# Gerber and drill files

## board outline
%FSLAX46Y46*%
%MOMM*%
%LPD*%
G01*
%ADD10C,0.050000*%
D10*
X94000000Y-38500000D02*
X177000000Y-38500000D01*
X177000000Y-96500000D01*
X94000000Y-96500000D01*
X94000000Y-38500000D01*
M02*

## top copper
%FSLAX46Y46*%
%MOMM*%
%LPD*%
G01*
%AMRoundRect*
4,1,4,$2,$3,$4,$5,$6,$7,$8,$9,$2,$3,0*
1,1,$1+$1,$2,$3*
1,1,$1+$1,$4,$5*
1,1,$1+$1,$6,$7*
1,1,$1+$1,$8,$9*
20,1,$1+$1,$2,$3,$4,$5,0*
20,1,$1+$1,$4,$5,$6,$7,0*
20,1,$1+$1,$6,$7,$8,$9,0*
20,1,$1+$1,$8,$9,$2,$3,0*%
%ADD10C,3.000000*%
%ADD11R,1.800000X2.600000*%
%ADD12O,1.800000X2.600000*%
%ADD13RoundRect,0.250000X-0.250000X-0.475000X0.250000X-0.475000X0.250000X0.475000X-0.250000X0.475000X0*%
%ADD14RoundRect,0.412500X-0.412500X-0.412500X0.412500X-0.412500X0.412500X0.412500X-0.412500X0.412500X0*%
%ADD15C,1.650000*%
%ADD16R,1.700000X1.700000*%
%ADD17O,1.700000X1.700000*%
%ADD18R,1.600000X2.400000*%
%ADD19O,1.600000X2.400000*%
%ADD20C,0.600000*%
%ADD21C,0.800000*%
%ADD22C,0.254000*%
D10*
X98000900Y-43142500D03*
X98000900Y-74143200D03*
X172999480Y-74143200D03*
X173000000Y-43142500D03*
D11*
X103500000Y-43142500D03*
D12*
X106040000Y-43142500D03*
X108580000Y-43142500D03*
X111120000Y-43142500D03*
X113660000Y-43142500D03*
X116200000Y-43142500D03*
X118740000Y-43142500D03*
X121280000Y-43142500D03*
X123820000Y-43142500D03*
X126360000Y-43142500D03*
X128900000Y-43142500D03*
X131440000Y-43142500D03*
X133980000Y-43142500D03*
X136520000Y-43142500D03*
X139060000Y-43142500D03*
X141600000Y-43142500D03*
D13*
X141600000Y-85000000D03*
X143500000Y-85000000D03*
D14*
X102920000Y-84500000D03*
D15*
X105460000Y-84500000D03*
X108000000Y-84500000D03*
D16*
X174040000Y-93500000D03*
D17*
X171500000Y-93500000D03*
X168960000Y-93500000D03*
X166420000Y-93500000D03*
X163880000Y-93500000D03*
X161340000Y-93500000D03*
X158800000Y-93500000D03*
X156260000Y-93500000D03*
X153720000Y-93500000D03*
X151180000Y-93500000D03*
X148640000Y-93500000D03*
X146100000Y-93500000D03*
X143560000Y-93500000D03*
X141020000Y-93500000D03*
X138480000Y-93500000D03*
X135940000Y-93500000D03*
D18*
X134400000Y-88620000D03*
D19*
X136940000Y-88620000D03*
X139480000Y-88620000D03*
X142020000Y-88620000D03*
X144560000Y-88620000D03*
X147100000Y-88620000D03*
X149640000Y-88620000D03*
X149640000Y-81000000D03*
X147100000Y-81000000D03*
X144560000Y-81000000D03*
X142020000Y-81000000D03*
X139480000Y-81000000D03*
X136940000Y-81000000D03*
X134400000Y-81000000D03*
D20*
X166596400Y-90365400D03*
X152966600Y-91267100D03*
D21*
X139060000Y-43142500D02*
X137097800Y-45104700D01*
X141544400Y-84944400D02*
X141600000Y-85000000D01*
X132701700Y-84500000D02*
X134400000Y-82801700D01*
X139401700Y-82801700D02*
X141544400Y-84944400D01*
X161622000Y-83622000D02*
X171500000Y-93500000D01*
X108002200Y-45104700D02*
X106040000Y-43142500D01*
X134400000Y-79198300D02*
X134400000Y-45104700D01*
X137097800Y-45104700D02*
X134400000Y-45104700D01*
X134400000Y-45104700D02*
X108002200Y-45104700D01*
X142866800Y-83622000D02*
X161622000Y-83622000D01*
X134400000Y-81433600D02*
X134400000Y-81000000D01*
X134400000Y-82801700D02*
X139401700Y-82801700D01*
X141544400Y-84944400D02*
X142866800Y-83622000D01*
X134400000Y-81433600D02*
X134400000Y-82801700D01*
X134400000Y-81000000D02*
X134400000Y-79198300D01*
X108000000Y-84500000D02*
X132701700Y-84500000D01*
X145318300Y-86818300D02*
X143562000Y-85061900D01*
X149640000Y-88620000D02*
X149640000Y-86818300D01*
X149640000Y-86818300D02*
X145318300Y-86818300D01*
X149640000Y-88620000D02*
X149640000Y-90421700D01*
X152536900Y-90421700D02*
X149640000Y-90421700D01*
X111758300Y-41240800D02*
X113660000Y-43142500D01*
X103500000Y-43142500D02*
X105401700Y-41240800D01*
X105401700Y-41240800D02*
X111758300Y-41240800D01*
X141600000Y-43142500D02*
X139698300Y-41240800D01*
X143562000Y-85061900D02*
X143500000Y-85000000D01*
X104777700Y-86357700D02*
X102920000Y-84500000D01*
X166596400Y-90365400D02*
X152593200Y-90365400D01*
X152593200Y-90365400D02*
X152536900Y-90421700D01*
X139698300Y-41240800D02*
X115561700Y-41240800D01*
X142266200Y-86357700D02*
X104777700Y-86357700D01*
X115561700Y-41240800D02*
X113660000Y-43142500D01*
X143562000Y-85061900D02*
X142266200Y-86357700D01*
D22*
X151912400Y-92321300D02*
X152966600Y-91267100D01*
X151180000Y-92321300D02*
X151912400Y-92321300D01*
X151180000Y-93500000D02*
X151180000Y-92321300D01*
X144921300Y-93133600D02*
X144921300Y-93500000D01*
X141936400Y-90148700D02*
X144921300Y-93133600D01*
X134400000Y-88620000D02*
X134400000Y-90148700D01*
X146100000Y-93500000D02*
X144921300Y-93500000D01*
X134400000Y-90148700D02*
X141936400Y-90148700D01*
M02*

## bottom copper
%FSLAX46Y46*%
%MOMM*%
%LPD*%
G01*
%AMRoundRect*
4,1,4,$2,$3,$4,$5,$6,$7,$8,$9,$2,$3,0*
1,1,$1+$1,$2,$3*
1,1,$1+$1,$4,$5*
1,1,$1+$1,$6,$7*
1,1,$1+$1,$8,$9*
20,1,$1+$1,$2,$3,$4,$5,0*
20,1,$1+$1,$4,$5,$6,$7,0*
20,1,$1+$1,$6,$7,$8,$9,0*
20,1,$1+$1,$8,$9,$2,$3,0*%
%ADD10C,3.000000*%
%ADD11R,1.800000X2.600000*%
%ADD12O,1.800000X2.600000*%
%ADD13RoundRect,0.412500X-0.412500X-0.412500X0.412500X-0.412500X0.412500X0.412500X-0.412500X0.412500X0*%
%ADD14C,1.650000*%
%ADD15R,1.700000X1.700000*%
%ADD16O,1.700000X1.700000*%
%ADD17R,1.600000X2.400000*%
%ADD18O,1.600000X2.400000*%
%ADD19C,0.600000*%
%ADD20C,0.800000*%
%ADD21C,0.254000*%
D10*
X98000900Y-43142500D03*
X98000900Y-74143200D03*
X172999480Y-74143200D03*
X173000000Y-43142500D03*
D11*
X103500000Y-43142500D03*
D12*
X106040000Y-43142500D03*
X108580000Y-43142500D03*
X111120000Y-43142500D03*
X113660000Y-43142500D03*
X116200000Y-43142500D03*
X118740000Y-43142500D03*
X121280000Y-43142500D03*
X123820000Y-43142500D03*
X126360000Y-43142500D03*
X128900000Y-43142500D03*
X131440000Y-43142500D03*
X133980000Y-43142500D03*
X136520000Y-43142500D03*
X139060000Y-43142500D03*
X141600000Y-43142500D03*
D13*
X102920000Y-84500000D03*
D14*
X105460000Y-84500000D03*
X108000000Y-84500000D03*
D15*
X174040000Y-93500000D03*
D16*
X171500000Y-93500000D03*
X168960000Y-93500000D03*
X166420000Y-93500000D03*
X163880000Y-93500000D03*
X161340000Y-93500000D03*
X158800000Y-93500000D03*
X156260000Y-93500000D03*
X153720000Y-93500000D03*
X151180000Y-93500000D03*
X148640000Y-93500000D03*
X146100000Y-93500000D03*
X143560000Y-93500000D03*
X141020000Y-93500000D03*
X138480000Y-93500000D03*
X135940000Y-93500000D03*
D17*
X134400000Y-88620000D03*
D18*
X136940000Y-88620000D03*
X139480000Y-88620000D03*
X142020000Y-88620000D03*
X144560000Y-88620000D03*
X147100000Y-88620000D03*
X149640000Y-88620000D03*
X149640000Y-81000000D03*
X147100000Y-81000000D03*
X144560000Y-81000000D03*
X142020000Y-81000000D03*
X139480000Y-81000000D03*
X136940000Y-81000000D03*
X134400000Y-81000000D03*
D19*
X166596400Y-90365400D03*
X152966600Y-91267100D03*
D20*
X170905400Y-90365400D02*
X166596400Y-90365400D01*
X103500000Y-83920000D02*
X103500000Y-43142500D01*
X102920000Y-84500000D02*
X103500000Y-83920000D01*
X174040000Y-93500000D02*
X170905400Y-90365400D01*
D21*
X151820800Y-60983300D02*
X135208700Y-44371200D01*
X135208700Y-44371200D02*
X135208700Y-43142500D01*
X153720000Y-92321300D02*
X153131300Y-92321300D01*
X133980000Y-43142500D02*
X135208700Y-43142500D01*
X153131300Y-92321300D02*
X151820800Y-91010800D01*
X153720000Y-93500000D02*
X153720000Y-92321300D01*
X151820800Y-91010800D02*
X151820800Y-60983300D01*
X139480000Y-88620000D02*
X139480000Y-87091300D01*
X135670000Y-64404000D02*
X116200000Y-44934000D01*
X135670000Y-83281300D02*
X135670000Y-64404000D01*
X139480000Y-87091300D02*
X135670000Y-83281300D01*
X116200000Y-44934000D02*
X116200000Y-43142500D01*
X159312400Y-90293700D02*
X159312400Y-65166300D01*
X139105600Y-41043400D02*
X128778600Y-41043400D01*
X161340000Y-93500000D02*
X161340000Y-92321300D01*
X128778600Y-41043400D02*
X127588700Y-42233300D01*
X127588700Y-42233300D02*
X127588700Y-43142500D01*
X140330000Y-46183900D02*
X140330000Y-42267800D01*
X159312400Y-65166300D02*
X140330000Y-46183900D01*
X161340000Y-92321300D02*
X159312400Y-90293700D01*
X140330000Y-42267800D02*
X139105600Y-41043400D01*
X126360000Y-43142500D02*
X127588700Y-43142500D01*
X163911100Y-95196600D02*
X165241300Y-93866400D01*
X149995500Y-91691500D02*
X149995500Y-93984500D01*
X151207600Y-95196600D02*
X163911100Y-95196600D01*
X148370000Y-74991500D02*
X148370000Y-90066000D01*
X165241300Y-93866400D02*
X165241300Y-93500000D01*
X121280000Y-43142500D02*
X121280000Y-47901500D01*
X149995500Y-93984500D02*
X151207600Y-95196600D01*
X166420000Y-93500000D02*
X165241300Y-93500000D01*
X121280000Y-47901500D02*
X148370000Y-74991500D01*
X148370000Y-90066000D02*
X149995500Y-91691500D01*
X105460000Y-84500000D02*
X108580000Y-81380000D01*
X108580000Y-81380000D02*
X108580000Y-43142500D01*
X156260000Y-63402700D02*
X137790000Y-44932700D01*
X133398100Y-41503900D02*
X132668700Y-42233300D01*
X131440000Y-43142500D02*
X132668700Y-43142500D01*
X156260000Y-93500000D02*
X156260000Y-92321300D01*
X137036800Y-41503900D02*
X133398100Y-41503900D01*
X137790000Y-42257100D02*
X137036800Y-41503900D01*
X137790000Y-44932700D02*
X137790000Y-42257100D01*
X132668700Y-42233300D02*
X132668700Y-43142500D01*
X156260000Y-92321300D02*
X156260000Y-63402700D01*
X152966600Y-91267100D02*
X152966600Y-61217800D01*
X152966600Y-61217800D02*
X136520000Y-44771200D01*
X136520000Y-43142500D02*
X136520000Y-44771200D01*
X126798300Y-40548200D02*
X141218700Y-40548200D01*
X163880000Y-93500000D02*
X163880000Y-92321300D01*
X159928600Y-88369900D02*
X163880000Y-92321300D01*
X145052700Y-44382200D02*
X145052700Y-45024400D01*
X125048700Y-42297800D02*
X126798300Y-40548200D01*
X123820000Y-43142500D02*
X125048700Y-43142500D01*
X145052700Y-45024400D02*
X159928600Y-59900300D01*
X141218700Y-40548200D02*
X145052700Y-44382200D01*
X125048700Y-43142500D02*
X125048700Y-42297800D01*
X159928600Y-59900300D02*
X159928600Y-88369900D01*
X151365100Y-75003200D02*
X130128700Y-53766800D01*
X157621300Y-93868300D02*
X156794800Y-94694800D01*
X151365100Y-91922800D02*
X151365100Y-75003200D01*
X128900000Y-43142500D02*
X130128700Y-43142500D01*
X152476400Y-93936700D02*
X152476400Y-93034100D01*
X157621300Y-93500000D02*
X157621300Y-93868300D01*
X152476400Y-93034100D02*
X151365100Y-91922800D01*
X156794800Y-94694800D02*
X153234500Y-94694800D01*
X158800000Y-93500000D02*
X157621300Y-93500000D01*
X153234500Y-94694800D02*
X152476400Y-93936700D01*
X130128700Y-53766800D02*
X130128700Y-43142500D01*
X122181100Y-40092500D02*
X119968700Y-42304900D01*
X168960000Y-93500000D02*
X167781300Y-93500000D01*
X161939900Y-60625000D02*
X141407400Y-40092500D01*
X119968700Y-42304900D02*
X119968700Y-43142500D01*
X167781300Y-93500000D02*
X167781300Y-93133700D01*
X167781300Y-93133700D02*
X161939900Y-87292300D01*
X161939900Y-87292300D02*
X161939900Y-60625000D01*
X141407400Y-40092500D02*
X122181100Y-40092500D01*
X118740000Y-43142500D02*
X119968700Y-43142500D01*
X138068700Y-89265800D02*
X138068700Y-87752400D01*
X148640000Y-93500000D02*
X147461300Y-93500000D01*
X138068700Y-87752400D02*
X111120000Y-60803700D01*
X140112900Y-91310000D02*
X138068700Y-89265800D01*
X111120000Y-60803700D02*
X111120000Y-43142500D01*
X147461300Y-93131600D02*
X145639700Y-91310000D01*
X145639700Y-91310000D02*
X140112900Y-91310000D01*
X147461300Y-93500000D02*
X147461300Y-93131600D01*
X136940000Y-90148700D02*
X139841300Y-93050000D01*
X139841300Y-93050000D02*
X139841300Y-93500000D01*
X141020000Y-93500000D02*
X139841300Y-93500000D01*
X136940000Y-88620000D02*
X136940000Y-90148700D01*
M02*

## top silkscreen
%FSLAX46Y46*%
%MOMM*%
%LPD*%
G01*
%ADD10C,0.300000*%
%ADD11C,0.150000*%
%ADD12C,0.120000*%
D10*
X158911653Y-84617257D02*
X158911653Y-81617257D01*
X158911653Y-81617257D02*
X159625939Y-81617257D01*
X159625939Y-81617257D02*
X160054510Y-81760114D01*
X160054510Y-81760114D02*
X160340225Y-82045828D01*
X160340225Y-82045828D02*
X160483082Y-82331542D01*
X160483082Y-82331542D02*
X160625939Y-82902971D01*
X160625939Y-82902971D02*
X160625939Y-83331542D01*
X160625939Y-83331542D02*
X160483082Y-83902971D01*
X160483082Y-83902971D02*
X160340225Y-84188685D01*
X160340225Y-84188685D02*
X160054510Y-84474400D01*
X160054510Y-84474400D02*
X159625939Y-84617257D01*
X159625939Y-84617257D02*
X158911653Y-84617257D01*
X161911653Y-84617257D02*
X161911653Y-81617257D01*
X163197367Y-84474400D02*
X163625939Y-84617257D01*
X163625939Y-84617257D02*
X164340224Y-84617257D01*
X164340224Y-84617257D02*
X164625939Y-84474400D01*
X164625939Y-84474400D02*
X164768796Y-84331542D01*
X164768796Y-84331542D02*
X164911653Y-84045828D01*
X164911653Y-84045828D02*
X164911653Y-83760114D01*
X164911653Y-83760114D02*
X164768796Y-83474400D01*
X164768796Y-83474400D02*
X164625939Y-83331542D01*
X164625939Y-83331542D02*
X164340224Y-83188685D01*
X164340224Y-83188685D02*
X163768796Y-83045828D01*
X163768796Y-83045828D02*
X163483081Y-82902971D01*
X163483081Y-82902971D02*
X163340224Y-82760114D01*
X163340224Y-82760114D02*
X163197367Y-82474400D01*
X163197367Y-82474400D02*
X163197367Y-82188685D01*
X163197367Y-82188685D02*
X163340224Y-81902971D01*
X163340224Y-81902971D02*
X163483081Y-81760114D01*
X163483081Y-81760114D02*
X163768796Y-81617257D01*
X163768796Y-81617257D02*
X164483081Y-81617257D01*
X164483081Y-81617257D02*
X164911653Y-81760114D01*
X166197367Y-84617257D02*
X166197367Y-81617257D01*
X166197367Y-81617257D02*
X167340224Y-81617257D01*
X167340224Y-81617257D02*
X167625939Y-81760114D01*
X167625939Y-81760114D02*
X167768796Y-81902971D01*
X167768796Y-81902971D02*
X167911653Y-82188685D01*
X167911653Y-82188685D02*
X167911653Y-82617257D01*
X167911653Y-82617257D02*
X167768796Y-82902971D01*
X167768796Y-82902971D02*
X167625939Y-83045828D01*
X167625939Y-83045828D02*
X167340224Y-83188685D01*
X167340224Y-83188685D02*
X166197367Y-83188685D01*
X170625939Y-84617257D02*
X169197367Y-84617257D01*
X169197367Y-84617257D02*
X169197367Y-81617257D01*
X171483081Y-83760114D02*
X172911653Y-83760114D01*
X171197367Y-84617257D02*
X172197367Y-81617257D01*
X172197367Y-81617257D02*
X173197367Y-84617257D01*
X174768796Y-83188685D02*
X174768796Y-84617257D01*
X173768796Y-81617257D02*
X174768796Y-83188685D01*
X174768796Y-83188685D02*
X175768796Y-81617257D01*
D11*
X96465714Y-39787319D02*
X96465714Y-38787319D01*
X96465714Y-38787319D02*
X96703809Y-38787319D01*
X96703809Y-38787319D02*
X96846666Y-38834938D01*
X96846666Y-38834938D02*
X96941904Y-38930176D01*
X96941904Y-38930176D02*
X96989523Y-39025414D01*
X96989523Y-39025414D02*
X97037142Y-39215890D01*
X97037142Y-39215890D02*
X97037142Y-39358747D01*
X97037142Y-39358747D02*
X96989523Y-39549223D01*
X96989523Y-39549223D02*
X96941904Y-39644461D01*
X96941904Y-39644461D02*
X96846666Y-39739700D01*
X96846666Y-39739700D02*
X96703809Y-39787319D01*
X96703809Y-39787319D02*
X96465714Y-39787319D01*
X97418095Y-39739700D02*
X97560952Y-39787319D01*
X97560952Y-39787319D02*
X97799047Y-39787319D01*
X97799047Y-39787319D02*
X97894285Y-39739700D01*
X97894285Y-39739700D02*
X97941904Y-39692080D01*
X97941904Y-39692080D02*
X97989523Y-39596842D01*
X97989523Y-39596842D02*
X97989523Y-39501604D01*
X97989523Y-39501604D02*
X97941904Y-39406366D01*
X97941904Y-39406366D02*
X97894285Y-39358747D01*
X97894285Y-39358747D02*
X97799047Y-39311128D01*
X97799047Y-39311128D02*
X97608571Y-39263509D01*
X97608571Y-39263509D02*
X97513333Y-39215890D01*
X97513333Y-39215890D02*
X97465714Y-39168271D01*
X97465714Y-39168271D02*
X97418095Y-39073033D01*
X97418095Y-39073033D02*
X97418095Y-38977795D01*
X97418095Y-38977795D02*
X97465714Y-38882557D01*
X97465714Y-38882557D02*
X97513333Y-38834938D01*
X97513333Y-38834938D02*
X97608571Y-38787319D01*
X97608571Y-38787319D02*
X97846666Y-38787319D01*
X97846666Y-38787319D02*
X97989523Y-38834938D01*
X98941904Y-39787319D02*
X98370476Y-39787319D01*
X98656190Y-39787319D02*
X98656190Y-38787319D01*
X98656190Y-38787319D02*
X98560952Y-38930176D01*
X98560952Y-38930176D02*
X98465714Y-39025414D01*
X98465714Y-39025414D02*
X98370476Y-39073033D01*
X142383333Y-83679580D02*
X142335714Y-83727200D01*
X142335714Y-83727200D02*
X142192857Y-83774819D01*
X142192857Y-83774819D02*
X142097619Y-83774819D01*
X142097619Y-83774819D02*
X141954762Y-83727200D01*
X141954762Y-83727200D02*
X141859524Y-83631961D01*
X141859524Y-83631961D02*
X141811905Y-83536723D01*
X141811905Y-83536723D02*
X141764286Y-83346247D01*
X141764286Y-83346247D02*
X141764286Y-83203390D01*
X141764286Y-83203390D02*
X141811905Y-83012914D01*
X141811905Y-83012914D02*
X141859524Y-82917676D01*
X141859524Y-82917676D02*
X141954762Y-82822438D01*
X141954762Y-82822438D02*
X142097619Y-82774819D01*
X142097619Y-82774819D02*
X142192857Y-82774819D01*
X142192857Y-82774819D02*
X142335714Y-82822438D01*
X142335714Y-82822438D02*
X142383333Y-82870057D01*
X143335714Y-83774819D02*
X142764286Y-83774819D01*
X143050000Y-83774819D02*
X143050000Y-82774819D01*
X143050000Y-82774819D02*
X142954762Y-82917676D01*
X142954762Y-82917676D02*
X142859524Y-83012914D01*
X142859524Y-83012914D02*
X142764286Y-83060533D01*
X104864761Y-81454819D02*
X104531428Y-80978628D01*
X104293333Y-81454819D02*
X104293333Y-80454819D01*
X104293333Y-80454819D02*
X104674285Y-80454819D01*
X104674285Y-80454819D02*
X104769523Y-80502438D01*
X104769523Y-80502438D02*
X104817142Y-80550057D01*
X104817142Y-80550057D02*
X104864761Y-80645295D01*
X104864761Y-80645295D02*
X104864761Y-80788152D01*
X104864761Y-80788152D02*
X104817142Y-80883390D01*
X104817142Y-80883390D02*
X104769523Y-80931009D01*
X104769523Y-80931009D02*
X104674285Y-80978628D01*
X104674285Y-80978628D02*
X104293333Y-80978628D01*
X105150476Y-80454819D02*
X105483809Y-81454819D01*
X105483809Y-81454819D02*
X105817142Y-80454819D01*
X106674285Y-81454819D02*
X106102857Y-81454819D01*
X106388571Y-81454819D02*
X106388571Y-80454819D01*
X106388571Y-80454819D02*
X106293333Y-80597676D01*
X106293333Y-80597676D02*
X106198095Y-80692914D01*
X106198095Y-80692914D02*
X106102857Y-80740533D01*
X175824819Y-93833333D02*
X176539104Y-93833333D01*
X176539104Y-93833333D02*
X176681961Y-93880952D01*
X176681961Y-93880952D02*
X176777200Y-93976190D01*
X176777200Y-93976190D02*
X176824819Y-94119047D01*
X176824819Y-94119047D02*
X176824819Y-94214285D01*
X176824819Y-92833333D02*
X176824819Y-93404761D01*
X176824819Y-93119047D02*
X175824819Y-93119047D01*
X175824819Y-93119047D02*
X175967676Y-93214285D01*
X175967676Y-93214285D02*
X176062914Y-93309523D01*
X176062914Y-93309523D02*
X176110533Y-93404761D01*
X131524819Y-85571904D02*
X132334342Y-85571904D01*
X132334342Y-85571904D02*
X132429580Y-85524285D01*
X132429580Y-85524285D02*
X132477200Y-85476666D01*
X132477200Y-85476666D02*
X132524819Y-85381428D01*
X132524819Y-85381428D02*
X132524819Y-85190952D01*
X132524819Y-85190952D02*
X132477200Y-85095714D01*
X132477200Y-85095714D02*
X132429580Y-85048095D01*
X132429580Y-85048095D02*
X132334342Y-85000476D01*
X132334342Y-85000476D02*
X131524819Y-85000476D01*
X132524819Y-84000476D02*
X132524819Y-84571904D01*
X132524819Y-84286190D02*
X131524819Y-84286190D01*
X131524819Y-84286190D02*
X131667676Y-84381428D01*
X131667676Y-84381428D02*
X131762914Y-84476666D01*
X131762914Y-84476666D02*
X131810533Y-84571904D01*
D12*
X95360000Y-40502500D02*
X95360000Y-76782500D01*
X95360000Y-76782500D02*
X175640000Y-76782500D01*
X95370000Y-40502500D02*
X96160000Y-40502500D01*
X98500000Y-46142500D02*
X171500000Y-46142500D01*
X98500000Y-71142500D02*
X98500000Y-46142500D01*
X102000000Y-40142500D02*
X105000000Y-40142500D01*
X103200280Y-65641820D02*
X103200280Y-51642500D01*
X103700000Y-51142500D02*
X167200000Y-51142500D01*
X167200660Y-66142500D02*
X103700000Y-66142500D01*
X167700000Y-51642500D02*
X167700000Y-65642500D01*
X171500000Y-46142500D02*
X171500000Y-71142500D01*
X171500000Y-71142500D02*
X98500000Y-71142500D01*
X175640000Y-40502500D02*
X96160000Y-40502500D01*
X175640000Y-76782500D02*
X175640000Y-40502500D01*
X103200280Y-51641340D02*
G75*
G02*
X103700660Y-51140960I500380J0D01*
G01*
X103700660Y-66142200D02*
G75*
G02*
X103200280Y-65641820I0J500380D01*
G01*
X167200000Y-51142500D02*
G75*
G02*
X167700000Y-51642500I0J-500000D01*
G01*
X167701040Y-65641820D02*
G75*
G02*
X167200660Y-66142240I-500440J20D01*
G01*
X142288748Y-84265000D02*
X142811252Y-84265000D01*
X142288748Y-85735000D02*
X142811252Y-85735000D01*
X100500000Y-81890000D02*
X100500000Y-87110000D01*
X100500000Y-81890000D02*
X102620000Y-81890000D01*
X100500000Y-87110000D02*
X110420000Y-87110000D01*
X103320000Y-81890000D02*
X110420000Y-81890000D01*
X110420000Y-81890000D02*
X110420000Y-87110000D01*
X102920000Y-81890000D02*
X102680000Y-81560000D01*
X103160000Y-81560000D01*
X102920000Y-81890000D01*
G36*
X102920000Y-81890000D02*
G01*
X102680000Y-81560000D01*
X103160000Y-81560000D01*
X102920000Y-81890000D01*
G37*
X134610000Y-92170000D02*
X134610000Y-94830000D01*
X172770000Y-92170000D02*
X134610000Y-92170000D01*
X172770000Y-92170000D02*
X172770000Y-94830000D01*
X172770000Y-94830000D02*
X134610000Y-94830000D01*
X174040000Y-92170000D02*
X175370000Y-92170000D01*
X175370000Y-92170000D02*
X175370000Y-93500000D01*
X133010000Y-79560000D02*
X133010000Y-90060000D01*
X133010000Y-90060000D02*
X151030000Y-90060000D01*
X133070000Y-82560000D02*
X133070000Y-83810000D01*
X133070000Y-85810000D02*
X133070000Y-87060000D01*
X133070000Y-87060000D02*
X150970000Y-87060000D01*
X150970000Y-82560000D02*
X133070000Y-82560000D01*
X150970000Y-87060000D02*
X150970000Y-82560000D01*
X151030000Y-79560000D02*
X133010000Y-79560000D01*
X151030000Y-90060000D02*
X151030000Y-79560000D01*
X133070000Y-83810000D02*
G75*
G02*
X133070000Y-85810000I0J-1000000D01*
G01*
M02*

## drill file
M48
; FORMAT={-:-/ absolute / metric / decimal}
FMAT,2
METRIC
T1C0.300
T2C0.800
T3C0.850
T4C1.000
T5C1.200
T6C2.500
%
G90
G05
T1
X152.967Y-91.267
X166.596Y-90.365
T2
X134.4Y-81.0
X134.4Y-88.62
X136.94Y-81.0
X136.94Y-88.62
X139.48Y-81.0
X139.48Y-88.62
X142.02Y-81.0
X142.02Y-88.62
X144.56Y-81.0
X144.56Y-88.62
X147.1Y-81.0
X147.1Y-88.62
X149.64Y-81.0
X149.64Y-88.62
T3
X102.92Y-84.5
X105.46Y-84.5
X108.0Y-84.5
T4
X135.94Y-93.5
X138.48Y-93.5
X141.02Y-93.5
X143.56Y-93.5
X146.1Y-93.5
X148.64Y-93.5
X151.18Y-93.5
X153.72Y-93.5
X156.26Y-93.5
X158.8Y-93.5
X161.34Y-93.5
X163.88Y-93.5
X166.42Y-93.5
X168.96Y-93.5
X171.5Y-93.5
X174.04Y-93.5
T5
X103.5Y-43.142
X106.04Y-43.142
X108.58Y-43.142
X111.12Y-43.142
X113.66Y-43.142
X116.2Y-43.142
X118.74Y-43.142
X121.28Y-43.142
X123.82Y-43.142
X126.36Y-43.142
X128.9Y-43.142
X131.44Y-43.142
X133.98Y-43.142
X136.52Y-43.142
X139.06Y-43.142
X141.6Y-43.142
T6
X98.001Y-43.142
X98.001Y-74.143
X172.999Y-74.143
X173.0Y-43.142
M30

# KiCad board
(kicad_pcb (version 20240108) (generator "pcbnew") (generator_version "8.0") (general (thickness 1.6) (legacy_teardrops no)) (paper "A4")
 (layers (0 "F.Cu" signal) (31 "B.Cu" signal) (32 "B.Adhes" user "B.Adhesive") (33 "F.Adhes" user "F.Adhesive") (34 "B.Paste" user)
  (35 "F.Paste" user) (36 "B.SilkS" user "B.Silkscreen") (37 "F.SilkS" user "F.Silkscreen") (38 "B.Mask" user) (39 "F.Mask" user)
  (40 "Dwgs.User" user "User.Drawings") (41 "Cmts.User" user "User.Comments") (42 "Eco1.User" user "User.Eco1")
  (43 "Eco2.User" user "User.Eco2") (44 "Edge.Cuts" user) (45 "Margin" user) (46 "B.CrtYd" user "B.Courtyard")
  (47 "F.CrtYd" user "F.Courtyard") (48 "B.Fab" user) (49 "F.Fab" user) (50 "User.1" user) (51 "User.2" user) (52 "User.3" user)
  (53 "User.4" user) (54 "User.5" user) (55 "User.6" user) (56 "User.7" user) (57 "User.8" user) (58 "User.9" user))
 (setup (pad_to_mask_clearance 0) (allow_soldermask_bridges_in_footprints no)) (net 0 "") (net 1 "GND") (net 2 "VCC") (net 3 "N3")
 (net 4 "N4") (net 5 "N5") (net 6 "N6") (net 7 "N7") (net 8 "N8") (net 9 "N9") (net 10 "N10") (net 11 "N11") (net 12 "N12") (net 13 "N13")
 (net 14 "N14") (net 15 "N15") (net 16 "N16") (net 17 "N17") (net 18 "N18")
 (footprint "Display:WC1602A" (layer "F.Cu") (at 103.5 43.1425)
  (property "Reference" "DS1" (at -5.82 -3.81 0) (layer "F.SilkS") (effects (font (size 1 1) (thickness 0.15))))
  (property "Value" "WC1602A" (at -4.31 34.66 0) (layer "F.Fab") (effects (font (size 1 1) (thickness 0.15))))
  (fp_line (start -8.14 -2.64) (end -8.14 33.64) (stroke (width 0.12) (type solid)) (layer "F.SilkS"))
  (fp_line (start -8.14 33.64) (end 72.14 33.64) (stroke (width 0.12) (type solid)) (layer "F.SilkS"))
  (fp_line (start -8.13 -2.64) (end -7.34 -2.64) (stroke (width 0.12) (type solid)) (layer "F.SilkS"))
  (fp_line (start -5 3) (end 68 3) (stroke (width 0.12) (type solid)) (layer "F.SilkS"))
  (fp_line (start -5 28) (end -5 3) (stroke (width 0.12) (type solid)) (layer "F.SilkS"))
  (fp_line (start -1.5 -3) (end 1.5 -3) (stroke (width 0.12) (type solid)) (layer "F.SilkS"))
  (fp_line (start -0.29972 22.49932) (end -0.29972 8.5) (stroke (width 0.12) (type solid)) (layer "F.SilkS"))
  (fp_line (start 0.2 8) (end 63.7 8) (stroke (width 0.12) (type solid)) (layer "F.SilkS"))
  (fp_line (start 63.70066 23) (end 0.2 23) (stroke (width 0.12) (type solid)) (layer "F.SilkS"))
  (fp_line (start 64.2 8.5) (end 64.2 22.5) (stroke (width 0.12) (type solid)) (layer "F.SilkS"))
  (fp_line (start 68 3) (end 68 28) (stroke (width 0.12) (type solid)) (layer "F.SilkS"))
  (fp_line (start 68 28) (end -5 28) (stroke (width 0.12) (type solid)) (layer "F.SilkS"))
  (fp_line (start 72.14 -2.64) (end -7.34 -2.64) (stroke (width 0.12) (type solid)) (layer "F.SilkS"))
  (fp_line (start 72.14 33.64) (end 72.14 -2.64) (stroke (width 0.12) (type solid)) (layer "F.SilkS"))
  (fp_arc (start -0.29972 8.49884) (mid -0.153162 8.145018) (end 0.20066 7.99846) (stroke (width 0.12) (type solid)) (layer "F.SilkS"))
  (fp_arc (start 0.20066 22.9997) (mid -0.153162 22.853142) (end -0.29972 22.49932) (stroke (width 0.12) (type solid)) (layer "F.SilkS"))
  (fp_arc (start 63.7 8) (mid 64.053553 8.146447) (end 64.2 8.5) (stroke (width 0.12) (type solid)) (layer "F.SilkS"))
  (fp_arc (start 64.20104 22.49932) (mid 64.054473 22.853115) (end 63.70066 22.9997) (stroke (width 0.12) (type solid)) (layer "F.SilkS"))
  (pad "" thru_hole circle (at -5.4991 0) (size 3 3) (drill 2.5) (layers "*.Cu" "*.Mask") (remove_unused_layers no))
  (pad "" thru_hole circle (at -5.4991 31.0007) (size 3 3) (drill 2.5) (layers "*.Cu" "*.Mask") (remove_unused_layers no))
  (pad "" thru_hole circle (at 69.49948 31.0007) (size 3 3) (drill 2.5) (layers "*.Cu" "*.Mask") (remove_unused_layers no))
  (pad "" thru_hole circle (at 69.5 0) (size 3 3) (drill 2.5) (layers "*.Cu" "*.Mask") (remove_unused_layers no))
  (pad "1" thru_hole rect (at 0 0) (size 1.8 2.6) (drill 1.2) (layers "*.Cu" "*.Mask") (remove_unused_layers no) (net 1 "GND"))
  (pad "2" thru_hole oval (at 2.54 0) (size 1.8 2.6) (drill 1.2) (layers "*.Cu" "*.Mask") (remove_unused_layers no) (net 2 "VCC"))
  (pad "3" thru_hole oval (at 5.08 0) (size 1.8 2.6) (drill 1.2) (layers "*.Cu" "*.Mask") (remove_unused_layers no) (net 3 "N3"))
  (pad "4" thru_hole oval (at 7.62 0) (size 1.8 2.6) (drill 1.2) (layers "*.Cu" "*.Mask") (remove_unused_layers no) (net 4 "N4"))
  (pad "5" thru_hole oval (at 10.16 0) (size 1.8 2.6) (drill 1.2) (layers "*.Cu" "*.Mask") (remove_unused_layers no) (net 1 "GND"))
  (pad "6" thru_hole oval (at 12.7 0) (size 1.8 2.6) (drill 1.2) (layers "*.Cu" "*.Mask") (remove_unused_layers no) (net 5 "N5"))
  (pad "7" thru_hole oval (at 15.24 0) (size 1.8 2.6) (drill 1.2) (layers "*.Cu" "*.Mask") (remove_unused_layers no) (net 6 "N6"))
  (pad "8" thru_hole oval (at 17.78 0) (size 1.8 2.6) (drill 1.2) (layers "*.Cu" "*.Mask") (remove_unused_layers no) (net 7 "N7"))
  (pad "9" thru_hole oval (at 20.32 0) (size 1.8 2.6) (drill 1.2) (layers "*.Cu" "*.Mask") (remove_unused_layers no) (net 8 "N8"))
  (pad "10" thru_hole oval (at 22.86 0) (size 1.8 2.6) (drill 1.2) (layers "*.Cu" "*.Mask") (remove_unused_layers no) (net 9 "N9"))
  (pad "11" thru_hole oval (at 25.4 0) (size 1.8 2.6) (drill 1.2) (layers "*.Cu" "*.Mask") (remove_unused_layers no) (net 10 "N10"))
  (pad "12" thru_hole oval (at 27.94 0) (size 1.8 2.6) (drill 1.2) (layers "*.Cu" "*.Mask") (remove_unused_layers no) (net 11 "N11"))
  (pad "13" thru_hole oval (at 30.48 0) (size 1.8 2.6) (drill 1.2) (layers "*.Cu" "*.Mask") (remove_unused_layers no) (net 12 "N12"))
  (pad "14" thru_hole oval (at 33.02 0) (size 1.8 2.6) (drill 1.2) (layers "*.Cu" "*.Mask") (remove_unused_layers no) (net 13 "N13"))
  (pad "15" thru_hole oval (at 35.56 0) (size 1.8 2.6) (drill 1.2) (layers "*.Cu" "*.Mask") (remove_unused_layers no) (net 2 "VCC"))
  (pad "16" thru_hole oval (at 38.1 0) (size 1.8 2.6) (drill 1.2) (layers "*.Cu" "*.Mask") (remove_unused_layers no) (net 1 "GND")))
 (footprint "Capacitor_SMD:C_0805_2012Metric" (layer "F.Cu") (at 142.55 85)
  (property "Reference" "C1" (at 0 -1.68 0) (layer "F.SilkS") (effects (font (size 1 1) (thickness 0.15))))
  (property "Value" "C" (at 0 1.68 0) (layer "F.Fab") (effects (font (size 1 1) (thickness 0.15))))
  (fp_line (start -0.261252 -0.735) (end 0.261252 -0.735) (stroke (width 0.12) (type solid)) (layer "F.SilkS"))
  (fp_line (start -0.261252 0.735) (end 0.261252 0.735) (stroke (width 0.12) (type solid)) (layer "F.SilkS"))
  (pad "1" smd roundrect (at -0.95 0) (size 1 1.45) (layers "F.Cu" "F.Paste" "F.Mask") (roundrect_rratio 0.25) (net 2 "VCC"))
  (pad "2" smd roundrect (at 0.95 0) (size 1 1.45) (layers "F.Cu" "F.Paste" "F.Mask") (roundrect_rratio 0.25) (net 1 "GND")))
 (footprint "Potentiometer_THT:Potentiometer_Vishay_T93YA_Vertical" (layer "F.Cu") (at 102.92 84.5)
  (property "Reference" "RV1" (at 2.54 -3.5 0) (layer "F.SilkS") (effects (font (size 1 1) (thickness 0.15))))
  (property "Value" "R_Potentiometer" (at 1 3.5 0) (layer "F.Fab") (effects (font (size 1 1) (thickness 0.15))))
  (fp_line (start -2.42 -2.61) (end -2.42 2.61) (stroke (width 0.12) (type default)) (layer "F.SilkS"))
  (fp_line (start -2.42 -2.61) (end -0.3 -2.61) (stroke (width 0.12) (type default)) (layer "F.SilkS"))
  (fp_line (start -2.42 2.61) (end 7.5 2.61) (stroke (width 0.12) (type default)) (layer "F.SilkS"))
  (fp_line (start 0.4 -2.61) (end 7.5 -2.61) (stroke (width 0.12) (type default)) (layer "F.SilkS"))
  (fp_line (start 7.5 -2.61) (end 7.5 2.61) (stroke (width 0.12) (type default)) (layer "F.SilkS"))
  (fp_poly
   (pts (xy 0 -2.61) (xy -0.24 -2.94) (xy 0.24 -2.94) (xy 0 -2.61)) (stroke (width 0.12) (type solid)) (fill solid) (layer "F.SilkS"))
  (pad "1" thru_hole roundrect (at 0 0) (size 1.65 1.65) (drill 0.85) (layers "*.Cu" "*.Mask") (remove_unused_layers no)
   (roundrect_rratio 0.25) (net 1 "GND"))
  (pad "2" thru_hole circle (at 2.54 0) (size 1.65 1.65) (drill 0.85) (layers "*.Cu" "*.Mask") (remove_unused_layers no) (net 3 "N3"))
  (pad "3" thru_hole circle (at 5.08 0) (size 1.65 1.65) (drill 0.85) (layers "*.Cu" "*.Mask") (remove_unused_layers no) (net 2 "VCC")))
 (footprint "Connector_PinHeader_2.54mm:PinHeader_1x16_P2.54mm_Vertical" (layer "F.Cu") (at 174.04 93.5 -90)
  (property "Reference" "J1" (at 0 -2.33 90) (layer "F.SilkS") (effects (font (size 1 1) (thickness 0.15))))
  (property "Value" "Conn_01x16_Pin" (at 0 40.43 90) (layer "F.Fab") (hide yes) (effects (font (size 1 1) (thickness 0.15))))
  (fp_line (start -1.33 39.43) (end 1.33 39.43) (stroke (width 0.12) (type solid)) (layer "F.SilkS"))
  (fp_line (start -1.33 1.27) (end -1.33 39.43) (stroke (width 0.12) (type solid)) (layer "F.SilkS"))
  (fp_line (start -1.33 1.27) (end 1.33 1.27) (stroke (width 0.12) (type solid)) (layer "F.SilkS"))
  (fp_line (start 1.33 1.27) (end 1.33 39.43) (stroke (width 0.12) (type solid)) (layer "F.SilkS"))
  (fp_line (start -1.33 0) (end -1.33 -1.33) (stroke (width 0.12) (type solid)) (layer "F.SilkS"))
  (fp_line (start -1.33 -1.33) (end 0 -1.33) (stroke (width 0.12) (type solid)) (layer "F.SilkS"))
  (pad "1" thru_hole rect (at 0 0 270) (size 1.7 1.7) (drill 1) (layers "*.Cu" "*.Mask") (remove_unused_layers no) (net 1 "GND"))
  (pad "2" thru_hole oval (at 0 2.54 270) (size 1.7 1.7) (drill 1) (layers "*.Cu" "*.Mask") (remove_unused_layers no) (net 2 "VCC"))
  (pad "3" thru_hole oval (at 0 5.08 270) (size 1.7 1.7) (drill 1) (layers "*.Cu" "*.Mask") (remove_unused_layers no) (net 6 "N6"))
  (pad "4" thru_hole oval (at 0 7.62 270) (size 1.7 1.7) (drill 1) (layers "*.Cu" "*.Mask") (remove_unused_layers no) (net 7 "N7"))
  (pad "5" thru_hole oval (at 0 10.16 270) (size 1.7 1.7) (drill 1) (layers "*.Cu" "*.Mask") (remove_unused_layers no) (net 8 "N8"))
  (pad "6" thru_hole oval (at 0 12.7 270) (size 1.7 1.7) (drill 1) (layers "*.Cu" "*.Mask") (remove_unused_layers no) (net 9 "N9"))
  (pad "7" thru_hole oval (at 0 15.24 270) (size 1.7 1.7) (drill 1) (layers "*.Cu" "*.Mask") (remove_unused_layers no) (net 10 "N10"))
  (pad "8" thru_hole oval (at 0 17.78 270) (size 1.7 1.7) (drill 1) (layers "*.Cu" "*.Mask") (remove_unused_layers no) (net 11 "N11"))
  (pad "9" thru_hole oval (at 0 20.32 270) (size 1.7 1.7) (drill 1) (layers "*.Cu" "*.Mask") (remove_unused_layers no) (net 12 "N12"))
  (pad "10" thru_hole oval (at 0 22.86 270) (size 1.7 1.7) (drill 1) (layers "*.Cu" "*.Mask") (remove_unused_layers no) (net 13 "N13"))
  (pad "11" thru_hole oval (at 0 25.4 270) (size 1.7 1.7) (drill 1) (layers "*.Cu" "*.Mask") (remove_unused_layers no) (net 4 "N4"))
  (pad "12" thru_hole oval (at 0 27.94 270) (size 1.7 1.7) (drill 1) (layers "*.Cu" "*.Mask") (remove_unused_layers no) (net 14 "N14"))
  (pad "13" thru_hole oval (at 0 30.48 270) (size 1.7 1.7) (drill 1) (layers "*.Cu" "*.Mask") (remove_unused_layers no) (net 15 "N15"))
  (pad "14" thru_hole oval (at 0 33.02 270) (size 1.7 1.7) (drill 1) (layers "*.Cu" "*.Mask") (remove_unused_layers no) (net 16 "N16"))
  (pad "15" thru_hole oval (at 0 35.56 270) (size 1.7 1.7) (drill 1) (layers "*.Cu" "*.Mask") (remove_unused_layers no) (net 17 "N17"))
  (pad "16" thru_hole oval (at 0 38.1 270) (size 1.7 1.7) (drill 1) (layers "*.Cu" "*.Mask") (remove_unused_layers no) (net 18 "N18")))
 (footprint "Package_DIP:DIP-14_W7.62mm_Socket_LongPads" (layer "F.Cu") (at 134.4 88.62 90)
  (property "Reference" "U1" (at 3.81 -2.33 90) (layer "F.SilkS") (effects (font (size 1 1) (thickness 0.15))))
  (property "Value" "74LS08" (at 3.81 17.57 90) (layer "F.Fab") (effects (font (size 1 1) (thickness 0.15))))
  (fp_line (start 9.06 -1.39) (end -1.44 -1.39) (stroke (width 0.12) (type solid)) (layer "F.SilkS"))
  (fp_line (start -1.44 -1.39) (end -1.44 16.63) (stroke (width 0.12) (type solid)) (layer "F.SilkS"))
  (fp_line (start 6.06 -1.33) (end 4.81 -1.33) (stroke (width 0.12) (type solid)) (layer "F.SilkS"))
  (fp_line (start 2.81 -1.33) (end 1.56 -1.33) (stroke (width 0.12) (type solid)) (layer "F.SilkS"))
  (fp_line (start 1.56 -1.33) (end 1.56 16.57) (stroke (width 0.12) (type solid)) (layer "F.SilkS"))
  (fp_line (start 6.06 16.57) (end 6.06 -1.33) (stroke (width 0.12) (type solid)) (layer "F.SilkS"))
  (fp_line (start 1.56 16.57) (end 6.06 16.57) (stroke (width 0.12) (type solid)) (layer "F.SilkS"))
  (fp_line (start 9.06 16.63) (end 9.06 -1.39) (stroke (width 0.12) (type solid)) (layer "F.SilkS"))
  (fp_line (start -1.44 16.63) (end 9.06 16.63) (stroke (width 0.12) (type solid)) (layer "F.SilkS"))
  (fp_arc (start 4.81 -1.33) (mid 3.81 -0.33) (end 2.81 -1.33) (stroke (width 0.12) (type solid)) (layer "F.SilkS"))
  (pad "1" thru_hole rect (at 0 0 90) (size 2.4 1.6) (drill 0.8) (layers "*.Cu" "*.Mask") (remove_unused_layers no) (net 14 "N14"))
  (pad "2" thru_hole oval (at 0 2.54 90) (size 2.4 1.6) (drill 0.8) (layers "*.Cu" "*.Mask") (remove_unused_layers no) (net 16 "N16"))
  (pad "3" thru_hole oval (at 0 5.08 90) (size 2.4 1.6) (drill 0.8) (layers "*.Cu" "*.Mask") (remove_unused_layers no) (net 5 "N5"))
  (pad "4" thru_hole oval (at 0 7.62 90) (size 2.4 1.6) (drill 0.8) (layers "*.Cu" "*.Mask") (remove_unused_layers no))
  (pad "5" thru_hole oval (at 0 10.16 90) (size 2.4 1.6) (drill 0.8) (layers "*.Cu" "*.Mask") (remove_unused_layers no))
  (pad "6" thru_hole oval (at 0 12.7 90) (size 2.4 1.6) (drill 0.8) (layers "*.Cu" "*.Mask") (remove_unused_layers no))
  (pad "7" thru_hole oval (at 0 15.24 90) (size 2.4 1.6) (drill 0.8) (layers "*.Cu" "*.Mask") (remove_unused_layers no) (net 1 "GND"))
  (pad "8" thru_hole oval (at 7.62 15.24 90) (size 2.4 1.6) (drill 0.8) (layers "*.Cu" "*.Mask") (remove_unused_layers no))
  (pad "9" thru_hole oval (at 7.62 12.7 90) (size 2.4 1.6) (drill 0.8) (layers "*.Cu" "*.Mask") (remove_unused_layers no))
  (pad "10" thru_hole oval (at 7.62 10.16 90) (size 2.4 1.6) (drill 0.8) (layers "*.Cu" "*.Mask") (remove_unused_layers no))
  (pad "11" thru_hole oval (at 7.62 7.62 90) (size 2.4 1.6) (drill 0.8) (layers "*.Cu" "*.Mask") (remove_unused_layers no))
  (pad "12" thru_hole oval (at 7.62 5.08 90) (size 2.4 1.6) (drill 0.8) (layers "*.Cu" "*.Mask") (remove_unused_layers no))
  (pad "13" thru_hole oval (at 7.62 2.54 90) (size 2.4 1.6) (drill 0.8) (layers "*.Cu" "*.Mask") (remove_unused_layers no))
  (pad "14" thru_hole oval (at 7.62 0 90) (size 2.4 1.6) (drill 0.8) (layers "*.Cu" "*.Mask") (remove_unused_layers no) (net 2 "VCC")))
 (gr_rect (start 94 38.5) (end 177 96.5) (stroke (width 0.05) (type default)) (fill none) (layer "Edge.Cuts"))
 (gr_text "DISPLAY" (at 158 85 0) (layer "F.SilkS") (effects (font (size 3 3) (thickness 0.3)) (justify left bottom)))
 (segment (start 139.06 43.1425) (end 137.0978 45.1047) (width 0.8) (layer "F.Cu") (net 2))
 (segment (start 141.5444 84.9444) (end 141.6 85) (width 0.8) (layer "F.Cu") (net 2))
 (segment (start 132.7017 84.5) (end 134.4 82.8017) (width 0.8) (layer "F.Cu") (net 2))
 (segment (start 139.4017 82.8017) (end 141.5444 84.9444) (width 0.8) (layer "F.Cu") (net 2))
 (segment (start 161.622 83.622) (end 171.5 93.5) (width 0.8) (layer "F.Cu") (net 2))
 (segment (start 108.0022 45.1047) (end 106.04 43.1425) (width 0.8) (layer "F.Cu") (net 2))
 (segment (start 134.4 79.1983) (end 134.4 45.1047) (width 0.8) (layer "F.Cu") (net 2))
 (segment (start 137.0978 45.1047) (end 134.4 45.1047) (width 0.8) (layer "F.Cu") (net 2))
 (segment (start 134.4 45.1047) (end 108.0022 45.1047) (width 0.8) (layer "F.Cu") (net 2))
 (segment (start 142.8668 83.622) (end 161.622 83.622) (width 0.8) (layer "F.Cu") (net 2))
 (segment (start 134.4 81.4336) (end 134.4 81) (width 0.8) (layer "F.Cu") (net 2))
 (segment (start 134.4 82.8017) (end 139.4017 82.8017) (width 0.8) (layer "F.Cu") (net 2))
 (segment (start 141.5444 84.9444) (end 142.8668 83.622) (width 0.8) (layer "F.Cu") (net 2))
 (segment (start 134.4 81.4336) (end 134.4 82.8017) (width 0.8) (layer "F.Cu") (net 2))
 (segment (start 134.4 81) (end 134.4 79.1983) (width 0.8) (layer "F.Cu") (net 2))
 (segment (start 108 84.5) (end 132.7017 84.5) (width 0.8) (layer "F.Cu") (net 2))
 (segment (start 145.3183 86.8183) (end 143.562 85.0619) (width 0.8) (layer "F.Cu") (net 1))
 (segment (start 149.64 88.62) (end 149.64 86.8183) (width 0.8) (layer "F.Cu") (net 1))
 (segment (start 149.64 86.8183) (end 145.3183 86.8183) (width 0.8) (layer "F.Cu") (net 1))
 (segment (start 149.64 88.62) (end 149.64 90.4217) (width 0.8) (layer "F.Cu") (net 1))
 (segment (start 152.5369 90.4217) (end 149.64 90.4217) (width 0.8) (layer "F.Cu") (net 1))
 (segment (start 111.7583 41.2408) (end 113.66 43.1425) (width 0.8) (layer "F.Cu") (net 1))
 (segment (start 103.5 43.1425) (end 105.4017 41.2408) (width 0.8) (layer "F.Cu") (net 1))
 (segment (start 105.4017 41.2408) (end 111.7583 41.2408) (width 0.8) (layer "F.Cu") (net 1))
 (segment (start 141.6 43.1425) (end 139.6983 41.2408) (width 0.8) (layer "F.Cu") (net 1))
 (segment (start 143.562 85.0619) (end 143.5 85) (width 0.8) (layer "F.Cu") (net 1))
 (segment (start 104.7777 86.3577) (end 102.92 84.5) (width 0.8) (layer "F.Cu") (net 1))
 (segment (start 166.5964 90.3654) (end 152.5932 90.3654) (width 0.8) (layer "F.Cu") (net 1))
 (segment (start 152.5932 90.3654) (end 152.5369 90.4217) (width 0.8) (layer "F.Cu") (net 1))
 (segment (start 139.6983 41.2408) (end 115.5617 41.2408) (width 0.8) (layer "F.Cu") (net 1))
 (segment (start 142.2662 86.3577) (end 104.7777 86.3577) (width 0.8) (layer "F.Cu") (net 1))
 (segment (start 115.5617 41.2408) (end 113.66 43.1425) (width 0.8) (layer "F.Cu") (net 1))
 (segment (start 143.562 85.0619) (end 142.2662 86.3577) (width 0.8) (layer "F.Cu") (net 1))
 (via (at 166.5964 90.3654) (size 0.6) (drill 0.3) (layers "F.Cu" "B.Cu") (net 1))
 (segment (start 170.9054 90.3654) (end 166.5964 90.3654) (width 0.8) (layer "B.Cu") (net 1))
 (segment (start 103.5 83.92) (end 103.5 43.1425) (width 0.8) (layer "B.Cu") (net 1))
 (segment (start 102.92 84.5) (end 103.5 83.92) (width 0.8) (layer "B.Cu") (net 1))
 (segment (start 174.04 93.5) (end 170.9054 90.3654) (width 0.8) (layer "B.Cu") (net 1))
 (segment (start 151.8208 60.9833) (end 135.2087 44.3712) (width 0.254) (layer "B.Cu") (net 12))
 (segment (start 135.2087 44.3712) (end 135.2087 43.1425) (width 0.254) (layer "B.Cu") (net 12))
 (segment (start 153.72 92.3213) (end 153.1313 92.3213) (width 0.254) (layer "B.Cu") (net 12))
 (segment (start 133.98 43.1425) (end 135.2087 43.1425) (width 0.254) (layer "B.Cu") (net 12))
 (segment (start 153.1313 92.3213) (end 151.8208 91.0108) (width 0.254) (layer "B.Cu") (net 12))
 (segment (start 153.72 93.5) (end 153.72 92.3213) (width 0.254) (layer "B.Cu") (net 12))
 (segment (start 151.8208 91.0108) (end 151.8208 60.9833) (width 0.254) (layer "B.Cu") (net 12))
 (segment (start 139.48 88.62) (end 139.48 87.0913) (width 0.254) (layer "B.Cu") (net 5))
 (segment (start 135.67 64.404) (end 116.2 44.934) (width 0.254) (layer "B.Cu") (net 5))
 (segment (start 135.67 83.2813) (end 135.67 64.404) (width 0.254) (layer "B.Cu") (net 5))
 (segment (start 139.48 87.0913) (end 135.67 83.2813) (width 0.254) (layer "B.Cu") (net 5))
 (segment (start 116.2 44.934) (end 116.2 43.1425) (width 0.254) (layer "B.Cu") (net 5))
 (segment (start 159.3124 90.2937) (end 159.3124 65.1663) (width 0.254) (layer "B.Cu") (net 9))
 (segment (start 139.1056 41.0434) (end 128.7786 41.0434) (width 0.254) (layer "B.Cu") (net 9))
 (segment (start 161.34 93.5) (end 161.34 92.3213) (width 0.254) (layer "B.Cu") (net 9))
 (segment (start 128.7786 41.0434) (end 127.5887 42.2333) (width 0.254) (layer "B.Cu") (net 9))
 (segment (start 127.5887 42.2333) (end 127.5887 43.1425) (width 0.254) (layer "B.Cu") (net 9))
 (segment (start 140.33 46.1839) (end 140.33 42.2678) (width 0.254) (layer "B.Cu") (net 9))
 (segment (start 159.3124 65.1663) (end 140.33 46.1839) (width 0.254) (layer "B.Cu") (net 9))
 (segment (start 161.34 92.3213) (end 159.3124 90.2937) (width 0.254) (layer "B.Cu") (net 9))
 (segment (start 140.33 42.2678) (end 139.1056 41.0434) (width 0.254) (layer "B.Cu") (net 9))
 (segment (start 126.36 43.1425) (end 127.5887 43.1425) (width 0.254) (layer "B.Cu") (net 9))
 (segment (start 163.9111 95.1966) (end 165.2413 93.8664) (width 0.254) (layer "B.Cu") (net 7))
 (segment (start 149.9955 91.6915) (end 149.9955 93.9845) (width 0.254) (layer "B.Cu") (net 7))
 (segment (start 151.2076 95.1966) (end 163.9111 95.1966) (width 0.254) (layer "B.Cu") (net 7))
 (segment (start 148.37 74.9915) (end 148.37 90.066) (width 0.254) (layer "B.Cu") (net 7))
 (segment (start 165.2413 93.8664) (end 165.2413 93.5) (width 0.254) (layer "B.Cu") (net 7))
 (segment (start 121.28 43.1425) (end 121.28 47.9015) (width 0.254) (layer "B.Cu") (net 7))
 (segment (start 149.9955 93.9845) (end 151.2076 95.1966) (width 0.254) (layer "B.Cu") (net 7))
 (segment (start 166.42 93.5) (end 165.2413 93.5) (width 0.254) (layer "B.Cu") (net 7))
 (segment (start 121.28 47.9015) (end 148.37 74.9915) (width 0.254) (layer "B.Cu") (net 7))
 (segment (start 148.37 90.066) (end 149.9955 91.6915) (width 0.254) (layer "B.Cu") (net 7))
 (segment (start 105.46 84.5) (end 108.58 81.38) (width 0.254) (layer "B.Cu") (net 3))
 (segment (start 108.58 81.38) (end 108.58 43.1425) (width 0.254) (layer "B.Cu") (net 3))
 (segment (start 156.26 63.4027) (end 137.79 44.9327) (width 0.254) (layer "B.Cu") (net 11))
 (segment (start 133.3981 41.5039) (end 132.6687 42.2333) (width 0.254) (layer "B.Cu") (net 11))
 (segment (start 131.44 43.1425) (end 132.6687 43.1425) (width 0.254) (layer "B.Cu") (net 11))
 (segment (start 156.26 93.5) (end 156.26 92.3213) (width 0.254) (layer "B.Cu") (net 11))
 (segment (start 137.0368 41.5039) (end 133.3981 41.5039) (width 0.254) (layer "B.Cu") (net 11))
 (segment (start 137.79 42.2571) (end 137.0368 41.5039) (width 0.254) (layer "B.Cu") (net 11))
 (segment (start 137.79 44.9327) (end 137.79 42.2571) (width 0.254) (layer "B.Cu") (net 11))
 (segment (start 132.6687 42.2333) (end 132.6687 43.1425) (width 0.254) (layer "B.Cu") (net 11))
 (segment (start 156.26 92.3213) (end 156.26 63.4027) (width 0.254) (layer "B.Cu") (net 11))
 (segment (start 151.9124 92.3213) (end 152.9666 91.2671) (width 0.254) (layer "F.Cu") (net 13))
 (segment (start 151.18 92.3213) (end 151.9124 92.3213) (width 0.254) (layer "F.Cu") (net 13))
 (segment (start 151.18 93.5) (end 151.18 92.3213) (width 0.254) (layer "F.Cu") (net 13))
 (via (at 152.9666 91.2671) (size 0.6) (drill 0.3) (layers "F.Cu" "B.Cu") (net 13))
 (segment (start 152.9666 91.2671) (end 152.9666 61.2178) (width 0.254) (layer "B.Cu") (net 13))
 (segment (start 152.9666 61.2178) (end 136.52 44.7712) (width 0.254) (layer "B.Cu") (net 13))
 (segment (start 136.52 43.1425) (end 136.52 44.7712) (width 0.254) (layer "B.Cu") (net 13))
 (segment (start 126.7983 40.5482) (end 141.2187 40.5482) (width 0.254) (layer "B.Cu") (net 8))
 (segment (start 163.88 93.5) (end 163.88 92.3213) (width 0.254) (layer "B.Cu") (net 8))
 (segment (start 159.9286 88.3699) (end 163.88 92.3213) (width 0.254) (layer "B.Cu") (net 8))
 (segment (start 145.0527 44.3822) (end 145.0527 45.0244) (width 0.254) (layer "B.Cu") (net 8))
 (segment (start 125.0487 42.2978) (end 126.7983 40.5482) (width 0.254) (layer "B.Cu") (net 8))
 (segment (start 123.82 43.1425) (end 125.0487 43.1425) (width 0.254) (layer "B.Cu") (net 8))
 (segment (start 145.0527 45.0244) (end 159.9286 59.9003) (width 0.254) (layer "B.Cu") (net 8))
 (segment (start 141.2187 40.5482) (end 145.0527 44.3822) (width 0.254) (layer "B.Cu") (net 8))
 (segment (start 125.0487 43.1425) (end 125.0487 42.2978) (width 0.254) (layer "B.Cu") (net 8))
 (segment (start 159.9286 59.9003) (end 159.9286 88.3699) (width 0.254) (layer "B.Cu") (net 8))
 (segment (start 151.3651 75.0032) (end 130.1287 53.7668) (width 0.254) (layer "B.Cu") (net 10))
 (segment (start 157.6213 93.8683) (end 156.7948 94.6948) (width 0.254) (layer "B.Cu") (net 10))
 (segment (start 151.3651 91.9228) (end 151.3651 75.0032) (width 0.254) (layer "B.Cu") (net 10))
 (segment (start 128.9 43.1425) (end 130.1287 43.1425) (width 0.254) (layer "B.Cu") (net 10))
 (segment (start 152.4764 93.9367) (end 152.4764 93.0341) (width 0.254) (layer "B.Cu") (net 10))
 (segment (start 157.6213 93.5) (end 157.6213 93.8683) (width 0.254) (layer "B.Cu") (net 10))
 (segment (start 152.4764 93.0341) (end 151.3651 91.9228) (width 0.254) (layer "B.Cu") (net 10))
 (segment (start 156.7948 94.6948) (end 153.2345 94.6948) (width 0.254) (layer "B.Cu") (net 10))
 (segment (start 158.8 93.5) (end 157.6213 93.5) (width 0.254) (layer "B.Cu") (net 10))
 (segment (start 153.2345 94.6948) (end 152.4764 93.9367) (width 0.254) (layer "B.Cu") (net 10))
 (segment (start 130.1287 53.7668) (end 130.1287 43.1425) (width 0.254) (layer "B.Cu") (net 10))
 (segment (start 122.1811 40.0925) (end 119.9687 42.3049) (width 0.254) (layer "B.Cu") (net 6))
 (segment (start 168.96 93.5) (end 167.7813 93.5) (width 0.254) (layer "B.Cu") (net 6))
 (segment (start 161.9399 60.625) (end 141.4074 40.0925) (width 0.254) (layer "B.Cu") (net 6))
 (segment (start 119.9687 42.3049) (end 119.9687 43.1425) (width 0.254) (layer "B.Cu") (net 6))
 (segment (start 167.7813 93.5) (end 167.7813 93.1337) (width 0.254) (layer "B.Cu") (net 6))
 (segment (start 167.7813 93.1337) (end 161.9399 87.2923) (width 0.254) (layer "B.Cu") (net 6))
 (segment (start 161.9399 87.2923) (end 161.9399 60.625) (width 0.254) (layer "B.Cu") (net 6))
 (segment (start 141.4074 40.0925) (end 122.1811 40.0925) (width 0.254) (layer "B.Cu") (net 6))
 (segment (start 118.74 43.1425) (end 119.9687 43.1425) (width 0.254) (layer "B.Cu") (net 6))
 (segment (start 138.0687 89.2658) (end 138.0687 87.7524) (width 0.254) (layer "B.Cu") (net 4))
 (segment (start 148.64 93.5) (end 147.4613 93.5) (width 0.254) (layer "B.Cu") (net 4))
 (segment (start 138.0687 87.7524) (end 111.12 60.8037) (width 0.254) (layer "B.Cu") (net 4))
 (segment (start 140.1129 91.31) (end 138.0687 89.2658) (width 0.254) (layer "B.Cu") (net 4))
 (segment (start 111.12 60.8037) (end 111.12 43.1425) (width 0.254) (layer "B.Cu") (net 4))
 (segment (start 147.4613 93.1316) (end 145.6397 91.31) (width 0.254) (layer "B.Cu") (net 4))
 (segment (start 145.6397 91.31) (end 140.1129 91.31) (width 0.254) (layer "B.Cu") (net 4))
 (segment (start 147.4613 93.5) (end 147.4613 93.1316) (width 0.254) (layer "B.Cu") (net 4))
 (segment (start 144.9213 93.1336) (end 144.9213 93.5) (width 0.254) (layer "F.Cu") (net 14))
 (segment (start 141.9364 90.1487) (end 144.9213 93.1336) (width 0.254) (layer "F.Cu") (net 14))
 (segment (start 134.4 88.62) (end 134.4 90.1487) (width 0.254) (layer "F.Cu") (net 14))
 (segment (start 146.1 93.5) (end 144.9213 93.5) (width 0.254) (layer "F.Cu") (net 14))
 (segment (start 134.4 90.1487) (end 141.9364 90.1487) (width 0.254) (layer "F.Cu") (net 14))
 (segment (start 136.94 90.1487) (end 139.8413 93.05) (width 0.254) (layer "B.Cu") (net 16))
 (segment (start 139.8413 93.05) (end 139.8413 93.5) (width 0.254) (layer "B.Cu") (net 16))
 (segment (start 141.02 93.5) (end 139.8413 93.5) (width 0.254) (layer "B.Cu") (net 16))
 (segment (start 136.94 88.62) (end 136.94 90.1487) (width 0.254) (layer "B.Cu") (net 16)))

